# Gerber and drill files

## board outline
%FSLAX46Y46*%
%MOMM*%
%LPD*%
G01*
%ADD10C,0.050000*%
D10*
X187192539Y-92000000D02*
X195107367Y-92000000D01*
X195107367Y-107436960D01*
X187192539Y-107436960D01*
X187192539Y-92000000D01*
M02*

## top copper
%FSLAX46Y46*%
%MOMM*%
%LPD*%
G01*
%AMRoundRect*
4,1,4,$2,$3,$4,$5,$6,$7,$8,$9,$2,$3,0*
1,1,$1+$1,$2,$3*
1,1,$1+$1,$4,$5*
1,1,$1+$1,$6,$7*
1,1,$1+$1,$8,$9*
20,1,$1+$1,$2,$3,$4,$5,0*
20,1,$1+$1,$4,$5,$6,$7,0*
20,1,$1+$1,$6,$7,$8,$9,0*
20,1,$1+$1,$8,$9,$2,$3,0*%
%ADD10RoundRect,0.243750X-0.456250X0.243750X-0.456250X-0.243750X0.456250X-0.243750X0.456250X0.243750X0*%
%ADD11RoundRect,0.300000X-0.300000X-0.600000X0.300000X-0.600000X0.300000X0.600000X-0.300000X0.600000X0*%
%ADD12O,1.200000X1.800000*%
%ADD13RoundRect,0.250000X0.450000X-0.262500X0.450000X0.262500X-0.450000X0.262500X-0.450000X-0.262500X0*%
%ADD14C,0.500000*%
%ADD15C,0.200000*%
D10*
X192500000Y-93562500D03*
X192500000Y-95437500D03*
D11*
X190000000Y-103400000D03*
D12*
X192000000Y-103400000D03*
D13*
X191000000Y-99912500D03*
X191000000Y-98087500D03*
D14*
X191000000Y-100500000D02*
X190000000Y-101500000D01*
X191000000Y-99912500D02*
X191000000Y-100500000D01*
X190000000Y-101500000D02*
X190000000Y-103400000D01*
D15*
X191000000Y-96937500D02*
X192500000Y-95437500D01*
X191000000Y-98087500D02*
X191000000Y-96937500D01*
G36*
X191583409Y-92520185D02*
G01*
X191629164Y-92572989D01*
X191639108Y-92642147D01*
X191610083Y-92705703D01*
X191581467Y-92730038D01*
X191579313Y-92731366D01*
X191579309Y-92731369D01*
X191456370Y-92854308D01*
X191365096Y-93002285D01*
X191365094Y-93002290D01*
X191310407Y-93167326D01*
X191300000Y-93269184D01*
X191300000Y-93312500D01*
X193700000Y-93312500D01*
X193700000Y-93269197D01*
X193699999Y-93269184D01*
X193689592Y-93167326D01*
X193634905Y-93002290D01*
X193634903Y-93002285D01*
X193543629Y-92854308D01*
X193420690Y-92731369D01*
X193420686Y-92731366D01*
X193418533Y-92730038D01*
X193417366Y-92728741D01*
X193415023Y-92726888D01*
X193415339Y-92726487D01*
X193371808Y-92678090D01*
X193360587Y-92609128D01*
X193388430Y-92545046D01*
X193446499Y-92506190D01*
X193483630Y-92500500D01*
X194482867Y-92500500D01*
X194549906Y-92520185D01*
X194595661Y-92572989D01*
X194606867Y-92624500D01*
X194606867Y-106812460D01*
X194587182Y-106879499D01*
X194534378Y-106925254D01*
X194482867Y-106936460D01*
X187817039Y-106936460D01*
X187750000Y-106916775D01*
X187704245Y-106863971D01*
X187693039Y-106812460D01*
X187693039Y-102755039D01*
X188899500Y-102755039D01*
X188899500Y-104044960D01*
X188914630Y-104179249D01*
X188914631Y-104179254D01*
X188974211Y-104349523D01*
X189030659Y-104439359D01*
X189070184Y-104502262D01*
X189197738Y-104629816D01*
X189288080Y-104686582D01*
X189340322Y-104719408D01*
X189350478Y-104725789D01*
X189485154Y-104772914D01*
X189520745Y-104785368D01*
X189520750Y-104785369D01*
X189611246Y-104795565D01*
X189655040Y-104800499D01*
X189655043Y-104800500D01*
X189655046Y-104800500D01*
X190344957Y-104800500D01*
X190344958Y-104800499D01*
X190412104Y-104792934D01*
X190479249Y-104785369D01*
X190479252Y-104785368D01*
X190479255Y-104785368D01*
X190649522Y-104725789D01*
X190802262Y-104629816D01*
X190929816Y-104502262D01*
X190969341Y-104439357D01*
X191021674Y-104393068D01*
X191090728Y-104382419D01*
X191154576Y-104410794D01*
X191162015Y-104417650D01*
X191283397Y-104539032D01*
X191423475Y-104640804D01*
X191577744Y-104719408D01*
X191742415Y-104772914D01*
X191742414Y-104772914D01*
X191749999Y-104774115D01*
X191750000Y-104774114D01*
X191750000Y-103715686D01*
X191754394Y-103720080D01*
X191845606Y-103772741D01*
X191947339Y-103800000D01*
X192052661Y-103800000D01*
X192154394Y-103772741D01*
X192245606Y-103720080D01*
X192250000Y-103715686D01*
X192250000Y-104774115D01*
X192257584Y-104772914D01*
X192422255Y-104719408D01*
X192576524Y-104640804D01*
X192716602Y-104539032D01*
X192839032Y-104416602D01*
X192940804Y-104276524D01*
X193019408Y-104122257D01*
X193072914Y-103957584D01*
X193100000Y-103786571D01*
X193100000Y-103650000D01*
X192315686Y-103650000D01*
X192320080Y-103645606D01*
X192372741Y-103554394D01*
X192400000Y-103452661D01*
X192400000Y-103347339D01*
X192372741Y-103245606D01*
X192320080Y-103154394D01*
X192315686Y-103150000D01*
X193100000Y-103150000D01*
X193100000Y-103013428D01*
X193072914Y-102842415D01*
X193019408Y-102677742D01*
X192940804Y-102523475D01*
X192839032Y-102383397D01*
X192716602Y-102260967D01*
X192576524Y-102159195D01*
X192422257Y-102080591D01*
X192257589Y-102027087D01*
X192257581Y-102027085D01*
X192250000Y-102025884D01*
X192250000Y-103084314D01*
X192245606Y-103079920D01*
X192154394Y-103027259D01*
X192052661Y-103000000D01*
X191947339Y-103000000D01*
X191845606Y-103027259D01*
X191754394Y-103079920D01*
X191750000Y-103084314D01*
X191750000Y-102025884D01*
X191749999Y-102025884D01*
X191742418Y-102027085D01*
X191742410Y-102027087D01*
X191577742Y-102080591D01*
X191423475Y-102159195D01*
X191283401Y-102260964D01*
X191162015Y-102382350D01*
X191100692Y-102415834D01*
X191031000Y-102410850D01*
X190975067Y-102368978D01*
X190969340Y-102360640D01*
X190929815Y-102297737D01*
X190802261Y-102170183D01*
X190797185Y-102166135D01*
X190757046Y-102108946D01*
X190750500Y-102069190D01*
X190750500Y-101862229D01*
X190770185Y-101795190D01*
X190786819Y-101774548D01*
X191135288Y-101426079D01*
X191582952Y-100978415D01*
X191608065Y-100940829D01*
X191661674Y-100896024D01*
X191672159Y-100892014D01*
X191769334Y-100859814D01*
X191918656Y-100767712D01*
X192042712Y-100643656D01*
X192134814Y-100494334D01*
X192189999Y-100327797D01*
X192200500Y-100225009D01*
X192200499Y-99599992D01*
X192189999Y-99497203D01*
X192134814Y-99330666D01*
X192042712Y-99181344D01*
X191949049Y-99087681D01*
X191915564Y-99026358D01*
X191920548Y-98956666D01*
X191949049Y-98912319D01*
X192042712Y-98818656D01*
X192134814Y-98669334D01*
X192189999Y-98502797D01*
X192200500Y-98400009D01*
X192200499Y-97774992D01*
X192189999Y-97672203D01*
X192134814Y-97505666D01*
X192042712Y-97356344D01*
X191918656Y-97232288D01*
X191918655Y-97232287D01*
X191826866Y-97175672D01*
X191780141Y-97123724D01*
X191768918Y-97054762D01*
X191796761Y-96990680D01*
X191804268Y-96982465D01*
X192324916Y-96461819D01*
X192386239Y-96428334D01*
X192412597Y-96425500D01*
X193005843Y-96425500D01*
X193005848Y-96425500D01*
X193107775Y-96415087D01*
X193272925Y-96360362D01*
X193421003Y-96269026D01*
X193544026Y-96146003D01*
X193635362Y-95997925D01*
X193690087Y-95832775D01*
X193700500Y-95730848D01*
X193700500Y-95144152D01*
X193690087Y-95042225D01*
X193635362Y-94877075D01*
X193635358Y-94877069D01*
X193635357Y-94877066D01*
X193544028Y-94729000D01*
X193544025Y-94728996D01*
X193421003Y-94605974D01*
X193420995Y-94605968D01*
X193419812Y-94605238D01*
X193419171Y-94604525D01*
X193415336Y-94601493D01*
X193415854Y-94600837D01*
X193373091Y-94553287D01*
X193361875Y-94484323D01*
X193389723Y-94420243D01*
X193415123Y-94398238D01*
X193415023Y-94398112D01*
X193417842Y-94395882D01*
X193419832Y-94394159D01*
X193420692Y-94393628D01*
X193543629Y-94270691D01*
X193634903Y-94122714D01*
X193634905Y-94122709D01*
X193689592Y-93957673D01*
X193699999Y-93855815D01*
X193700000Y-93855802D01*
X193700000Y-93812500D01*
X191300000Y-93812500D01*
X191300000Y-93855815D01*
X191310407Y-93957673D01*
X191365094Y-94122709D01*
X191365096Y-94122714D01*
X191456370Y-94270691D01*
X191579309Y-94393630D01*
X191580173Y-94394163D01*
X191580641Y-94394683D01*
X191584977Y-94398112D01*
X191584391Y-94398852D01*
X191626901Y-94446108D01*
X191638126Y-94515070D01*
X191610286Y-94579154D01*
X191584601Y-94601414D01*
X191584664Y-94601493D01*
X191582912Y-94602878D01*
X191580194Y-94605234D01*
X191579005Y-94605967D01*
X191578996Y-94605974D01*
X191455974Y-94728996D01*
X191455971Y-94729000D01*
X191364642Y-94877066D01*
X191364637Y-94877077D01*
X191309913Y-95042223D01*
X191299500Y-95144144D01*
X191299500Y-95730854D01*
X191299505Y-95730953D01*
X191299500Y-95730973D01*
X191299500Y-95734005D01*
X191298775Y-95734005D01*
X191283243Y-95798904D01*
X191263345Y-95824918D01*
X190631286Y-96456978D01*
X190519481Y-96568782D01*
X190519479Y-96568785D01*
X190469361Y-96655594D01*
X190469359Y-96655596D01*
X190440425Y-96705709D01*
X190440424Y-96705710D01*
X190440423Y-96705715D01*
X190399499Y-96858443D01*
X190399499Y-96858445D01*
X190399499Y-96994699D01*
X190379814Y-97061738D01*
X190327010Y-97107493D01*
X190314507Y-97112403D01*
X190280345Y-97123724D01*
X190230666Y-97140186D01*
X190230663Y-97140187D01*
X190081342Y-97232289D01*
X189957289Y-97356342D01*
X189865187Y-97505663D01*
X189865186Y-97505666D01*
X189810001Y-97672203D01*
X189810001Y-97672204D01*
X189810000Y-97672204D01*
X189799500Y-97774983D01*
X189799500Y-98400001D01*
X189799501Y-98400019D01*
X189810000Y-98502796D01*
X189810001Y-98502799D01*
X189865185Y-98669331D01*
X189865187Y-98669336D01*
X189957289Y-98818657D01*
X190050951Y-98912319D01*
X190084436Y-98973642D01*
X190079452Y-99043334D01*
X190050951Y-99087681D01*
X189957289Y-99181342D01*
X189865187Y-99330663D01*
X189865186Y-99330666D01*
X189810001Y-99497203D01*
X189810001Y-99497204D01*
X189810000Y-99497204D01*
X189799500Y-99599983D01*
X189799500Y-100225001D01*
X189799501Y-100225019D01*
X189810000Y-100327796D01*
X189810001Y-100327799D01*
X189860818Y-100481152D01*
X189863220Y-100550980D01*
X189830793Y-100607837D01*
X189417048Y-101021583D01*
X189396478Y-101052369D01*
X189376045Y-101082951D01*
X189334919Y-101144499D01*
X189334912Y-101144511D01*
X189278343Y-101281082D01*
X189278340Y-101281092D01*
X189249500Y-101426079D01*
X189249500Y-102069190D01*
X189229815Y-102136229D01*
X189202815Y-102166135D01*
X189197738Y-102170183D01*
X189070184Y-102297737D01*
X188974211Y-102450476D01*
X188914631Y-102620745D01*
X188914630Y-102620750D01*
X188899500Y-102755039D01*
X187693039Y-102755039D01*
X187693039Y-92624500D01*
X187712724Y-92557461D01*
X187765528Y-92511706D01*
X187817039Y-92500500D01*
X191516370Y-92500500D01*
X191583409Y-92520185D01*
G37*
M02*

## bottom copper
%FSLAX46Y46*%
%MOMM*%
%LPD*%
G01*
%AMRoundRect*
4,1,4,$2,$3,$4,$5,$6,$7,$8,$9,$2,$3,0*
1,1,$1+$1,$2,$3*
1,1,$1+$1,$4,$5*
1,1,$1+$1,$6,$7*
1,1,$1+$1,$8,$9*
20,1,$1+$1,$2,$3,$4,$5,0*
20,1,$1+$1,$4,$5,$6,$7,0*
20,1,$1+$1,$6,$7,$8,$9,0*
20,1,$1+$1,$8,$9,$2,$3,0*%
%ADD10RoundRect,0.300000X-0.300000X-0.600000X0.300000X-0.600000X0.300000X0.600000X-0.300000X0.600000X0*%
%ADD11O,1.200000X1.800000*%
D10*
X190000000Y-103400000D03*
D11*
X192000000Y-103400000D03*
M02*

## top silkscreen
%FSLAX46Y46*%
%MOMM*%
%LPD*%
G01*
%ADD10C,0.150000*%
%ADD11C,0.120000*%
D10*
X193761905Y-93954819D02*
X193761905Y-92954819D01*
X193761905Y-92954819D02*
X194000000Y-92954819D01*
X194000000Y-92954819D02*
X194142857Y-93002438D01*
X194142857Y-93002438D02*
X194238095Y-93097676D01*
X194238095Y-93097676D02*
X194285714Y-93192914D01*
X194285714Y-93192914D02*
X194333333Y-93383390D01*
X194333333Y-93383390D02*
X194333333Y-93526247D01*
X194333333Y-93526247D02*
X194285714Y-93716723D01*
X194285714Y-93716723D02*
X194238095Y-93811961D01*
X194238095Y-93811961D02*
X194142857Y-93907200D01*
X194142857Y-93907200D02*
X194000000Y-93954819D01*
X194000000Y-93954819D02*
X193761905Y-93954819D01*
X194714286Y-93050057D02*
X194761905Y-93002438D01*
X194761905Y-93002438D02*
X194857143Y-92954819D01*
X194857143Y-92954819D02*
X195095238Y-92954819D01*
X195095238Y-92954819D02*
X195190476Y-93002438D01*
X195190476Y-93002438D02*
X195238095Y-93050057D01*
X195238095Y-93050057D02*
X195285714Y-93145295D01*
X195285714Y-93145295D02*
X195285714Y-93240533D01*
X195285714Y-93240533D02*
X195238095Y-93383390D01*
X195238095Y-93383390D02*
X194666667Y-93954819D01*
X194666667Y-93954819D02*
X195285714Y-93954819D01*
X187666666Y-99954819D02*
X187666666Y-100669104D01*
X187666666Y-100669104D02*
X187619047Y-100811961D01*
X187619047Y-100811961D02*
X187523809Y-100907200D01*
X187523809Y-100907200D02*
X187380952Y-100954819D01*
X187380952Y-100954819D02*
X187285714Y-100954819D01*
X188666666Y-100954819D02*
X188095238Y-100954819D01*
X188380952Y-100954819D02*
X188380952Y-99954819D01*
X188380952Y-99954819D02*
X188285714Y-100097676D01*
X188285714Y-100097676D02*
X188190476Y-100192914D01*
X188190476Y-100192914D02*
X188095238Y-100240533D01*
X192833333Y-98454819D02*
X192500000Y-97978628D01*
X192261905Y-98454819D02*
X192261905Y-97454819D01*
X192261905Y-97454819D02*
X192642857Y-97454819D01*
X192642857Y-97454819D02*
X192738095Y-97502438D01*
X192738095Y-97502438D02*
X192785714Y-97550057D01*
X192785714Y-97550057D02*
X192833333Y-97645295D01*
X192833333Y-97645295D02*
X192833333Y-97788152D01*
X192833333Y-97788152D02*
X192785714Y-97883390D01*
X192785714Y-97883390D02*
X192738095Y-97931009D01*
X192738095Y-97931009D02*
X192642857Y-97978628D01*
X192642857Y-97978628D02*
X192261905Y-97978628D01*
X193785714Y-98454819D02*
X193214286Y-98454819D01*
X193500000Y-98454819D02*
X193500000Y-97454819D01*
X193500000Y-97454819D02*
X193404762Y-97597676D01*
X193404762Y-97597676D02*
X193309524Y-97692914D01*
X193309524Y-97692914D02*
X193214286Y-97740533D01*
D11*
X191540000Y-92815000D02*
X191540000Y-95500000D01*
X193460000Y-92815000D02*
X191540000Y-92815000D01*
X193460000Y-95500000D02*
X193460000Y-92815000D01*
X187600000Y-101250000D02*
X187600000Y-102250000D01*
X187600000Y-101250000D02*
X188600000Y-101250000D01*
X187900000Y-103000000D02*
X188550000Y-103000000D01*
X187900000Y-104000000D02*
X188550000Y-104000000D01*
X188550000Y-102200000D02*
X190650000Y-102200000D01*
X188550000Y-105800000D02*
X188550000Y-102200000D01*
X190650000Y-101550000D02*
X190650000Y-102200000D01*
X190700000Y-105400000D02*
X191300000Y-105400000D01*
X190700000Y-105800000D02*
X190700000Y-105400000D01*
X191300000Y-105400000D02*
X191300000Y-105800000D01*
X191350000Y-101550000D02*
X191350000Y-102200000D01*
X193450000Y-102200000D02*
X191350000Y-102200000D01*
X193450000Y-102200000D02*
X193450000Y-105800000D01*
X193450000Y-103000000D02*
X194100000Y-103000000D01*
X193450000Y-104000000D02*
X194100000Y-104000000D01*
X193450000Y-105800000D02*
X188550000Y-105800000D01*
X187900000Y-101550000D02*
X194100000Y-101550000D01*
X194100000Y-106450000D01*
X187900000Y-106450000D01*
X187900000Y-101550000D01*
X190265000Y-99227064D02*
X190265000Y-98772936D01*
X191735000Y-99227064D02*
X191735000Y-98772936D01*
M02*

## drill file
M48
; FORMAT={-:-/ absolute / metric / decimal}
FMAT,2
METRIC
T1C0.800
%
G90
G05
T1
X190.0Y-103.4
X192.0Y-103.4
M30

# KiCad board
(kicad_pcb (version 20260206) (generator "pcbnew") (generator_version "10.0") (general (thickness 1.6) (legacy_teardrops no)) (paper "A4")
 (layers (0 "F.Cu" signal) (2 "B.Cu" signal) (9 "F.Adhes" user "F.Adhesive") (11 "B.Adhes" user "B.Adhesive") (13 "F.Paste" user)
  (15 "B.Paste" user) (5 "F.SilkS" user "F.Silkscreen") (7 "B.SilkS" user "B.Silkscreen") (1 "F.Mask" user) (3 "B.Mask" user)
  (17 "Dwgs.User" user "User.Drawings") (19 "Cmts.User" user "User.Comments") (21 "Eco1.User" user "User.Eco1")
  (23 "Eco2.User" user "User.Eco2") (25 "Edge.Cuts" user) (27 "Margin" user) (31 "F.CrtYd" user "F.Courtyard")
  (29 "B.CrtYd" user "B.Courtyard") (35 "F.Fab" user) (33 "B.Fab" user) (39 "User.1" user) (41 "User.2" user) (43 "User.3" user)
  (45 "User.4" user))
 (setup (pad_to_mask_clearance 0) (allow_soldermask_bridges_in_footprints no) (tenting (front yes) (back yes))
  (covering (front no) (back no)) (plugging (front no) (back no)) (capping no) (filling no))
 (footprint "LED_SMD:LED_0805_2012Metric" (layer "F.Cu") (at 192.5 94.5 -90)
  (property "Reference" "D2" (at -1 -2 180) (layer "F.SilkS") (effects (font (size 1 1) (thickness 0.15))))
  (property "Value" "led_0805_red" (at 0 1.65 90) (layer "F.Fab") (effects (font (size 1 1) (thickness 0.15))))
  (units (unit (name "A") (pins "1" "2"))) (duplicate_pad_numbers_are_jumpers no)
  (fp_line (start -1.685 0.96) (end 1 0.96) (stroke (width 0.12) (type solid)) (layer "F.SilkS"))
  (fp_line (start -1.685 -0.96) (end -1.685 0.96) (stroke (width 0.12) (type solid)) (layer "F.SilkS"))
  (fp_line (start 1 -0.96) (end -1.685 -0.96) (stroke (width 0.12) (type solid)) (layer "F.SilkS"))
  (pad "1" smd roundrect (at -0.9375 0 270) (size 0.975 1.4) (layers "F.Cu" "F.Mask" "F.Paste") (roundrect_rratio 0.25) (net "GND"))
  (pad "2" smd roundrect (at 0.9375 0 270) (size 0.975 1.4) (layers "F.Cu" "F.Mask" "F.Paste") (roundrect_rratio 0.25) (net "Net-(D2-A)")))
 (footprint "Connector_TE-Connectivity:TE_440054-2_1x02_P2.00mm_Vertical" (layer "F.Cu") (at 190 103.4)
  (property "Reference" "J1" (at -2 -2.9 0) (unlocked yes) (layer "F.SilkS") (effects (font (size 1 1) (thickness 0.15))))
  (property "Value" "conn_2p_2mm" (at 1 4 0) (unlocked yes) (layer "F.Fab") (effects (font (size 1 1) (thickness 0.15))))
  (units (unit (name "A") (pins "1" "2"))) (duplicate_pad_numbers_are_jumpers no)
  (fp_line (start -2.4 -2.15) (end -2.4 -1.15) (stroke (width 0.12) (type solid)) (layer "F.SilkS"))
  (fp_line (start -2.4 -2.15) (end -1.4 -2.15) (stroke (width 0.12) (type solid)) (layer "F.SilkS"))
  (fp_line (start -2.1 -0.4) (end -1.45 -0.4) (stroke (width 0.12) (type solid)) (layer "F.SilkS"))
  (fp_line (start -2.1 0.6) (end -1.45 0.6) (stroke (width 0.12) (type solid)) (layer "F.SilkS"))
  (fp_line (start -1.45 -1.2) (end 0.65 -1.2) (stroke (width 0.12) (type solid)) (layer "F.SilkS"))
  (fp_line (start -1.45 2.4) (end -1.45 -1.2) (stroke (width 0.12) (type solid)) (layer "F.SilkS"))
  (fp_line (start 0.65 -1.85) (end 0.65 -1.2) (stroke (width 0.12) (type solid)) (layer "F.SilkS"))
  (fp_line (start 0.7 2) (end 1.3 2) (stroke (width 0.12) (type solid)) (layer "F.SilkS"))
  (fp_line (start 0.7 2.4) (end 0.7 2) (stroke (width 0.12) (type solid)) (layer "F.SilkS"))
  (fp_line (start 1.3 2) (end 1.3 2.4) (stroke (width 0.12) (type solid)) (layer "F.SilkS"))
  (fp_line (start 1.35 -1.85) (end 1.35 -1.2) (stroke (width 0.12) (type solid)) (layer "F.SilkS"))
  (fp_line (start 3.45 -1.2) (end 1.35 -1.2) (stroke (width 0.12) (type solid)) (layer "F.SilkS"))
  (fp_line (start 3.45 -1.2) (end 3.45 2.4) (stroke (width 0.12) (type solid)) (layer "F.SilkS"))
  (fp_line (start 3.45 -0.4) (end 4.1 -0.4) (stroke (width 0.12) (type solid)) (layer "F.SilkS"))
  (fp_line (start 3.45 0.6) (end 4.1 0.6) (stroke (width 0.12) (type solid)) (layer "F.SilkS"))
  (fp_line (start 3.45 2.4) (end -1.45 2.4) (stroke (width 0.12) (type solid)) (layer "F.SilkS"))
  (fp_rect (start -2.1 -1.85) (end 4.1 3.05) (stroke (width 0.12) (type solid)) (fill no) (layer "F.SilkS"))
  (pad "1" thru_hole roundrect (at 0 0) (size 1.2 1.8) (drill 0.8) (layers "*.Cu" "*.Mask") (remove_unused_layers no)
   (roundrect_rratio 0.25) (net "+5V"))
  (pad "2" thru_hole oval (at 2 0) (size 1.2 1.8) (drill 0.8) (layers "*.Cu" "*.Mask") (remove_unused_layers no) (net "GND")))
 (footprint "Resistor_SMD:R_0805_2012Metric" (layer "F.Cu") (at 191 99 90)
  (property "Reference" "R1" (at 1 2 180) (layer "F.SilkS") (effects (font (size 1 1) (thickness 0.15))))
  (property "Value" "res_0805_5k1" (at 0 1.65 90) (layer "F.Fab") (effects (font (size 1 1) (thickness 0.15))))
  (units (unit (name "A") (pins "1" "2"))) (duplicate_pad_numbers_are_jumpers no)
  (fp_line (start -0.227064 -0.735) (end 0.227064 -0.735) (stroke (width 0.12) (type solid)) (layer "F.SilkS"))
  (fp_line (start -0.227064 0.735) (end 0.227064 0.735) (stroke (width 0.12) (type solid)) (layer "F.SilkS"))
  (pad "1" smd roundrect (at -0.9125 0 90) (size 1.025 1.4) (layers "F.Cu" "F.Mask" "F.Paste") (roundrect_rratio 0.243902) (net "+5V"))
  (pad "2" smd roundrect (at 0.9125 0 90) (size 1.025 1.4) (layers "F.Cu" "F.Mask" "F.Paste") (roundrect_rratio 0.243902) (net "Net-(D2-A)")))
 (gr_rect (start 187.192539 92) (end 195.107367 107.43696) (stroke (width 0.05) (type default)) (fill no) (layer "Edge.Cuts"))
 (segment (start 191 100.5) (end 190 101.5) (width 0.5) (layer "F.Cu") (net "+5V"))
 (segment (start 191 99.9125) (end 191 100.5) (width 0.5) (layer "F.Cu") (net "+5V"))
 (segment (start 190 101.5) (end 190 103.4) (width 0.5) (layer "F.Cu") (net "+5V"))
 (segment (start 191 96.9375) (end 192.5 95.4375) (width 0.2) (layer "F.Cu") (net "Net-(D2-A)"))
 (segment (start 191 98.0875) (end 191 96.9375) (width 0.2) (layer "F.Cu") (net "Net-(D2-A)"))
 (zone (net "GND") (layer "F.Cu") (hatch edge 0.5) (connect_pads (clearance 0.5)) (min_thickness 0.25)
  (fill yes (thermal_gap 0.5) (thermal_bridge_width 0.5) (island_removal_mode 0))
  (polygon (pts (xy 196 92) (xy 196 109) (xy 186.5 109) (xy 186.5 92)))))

